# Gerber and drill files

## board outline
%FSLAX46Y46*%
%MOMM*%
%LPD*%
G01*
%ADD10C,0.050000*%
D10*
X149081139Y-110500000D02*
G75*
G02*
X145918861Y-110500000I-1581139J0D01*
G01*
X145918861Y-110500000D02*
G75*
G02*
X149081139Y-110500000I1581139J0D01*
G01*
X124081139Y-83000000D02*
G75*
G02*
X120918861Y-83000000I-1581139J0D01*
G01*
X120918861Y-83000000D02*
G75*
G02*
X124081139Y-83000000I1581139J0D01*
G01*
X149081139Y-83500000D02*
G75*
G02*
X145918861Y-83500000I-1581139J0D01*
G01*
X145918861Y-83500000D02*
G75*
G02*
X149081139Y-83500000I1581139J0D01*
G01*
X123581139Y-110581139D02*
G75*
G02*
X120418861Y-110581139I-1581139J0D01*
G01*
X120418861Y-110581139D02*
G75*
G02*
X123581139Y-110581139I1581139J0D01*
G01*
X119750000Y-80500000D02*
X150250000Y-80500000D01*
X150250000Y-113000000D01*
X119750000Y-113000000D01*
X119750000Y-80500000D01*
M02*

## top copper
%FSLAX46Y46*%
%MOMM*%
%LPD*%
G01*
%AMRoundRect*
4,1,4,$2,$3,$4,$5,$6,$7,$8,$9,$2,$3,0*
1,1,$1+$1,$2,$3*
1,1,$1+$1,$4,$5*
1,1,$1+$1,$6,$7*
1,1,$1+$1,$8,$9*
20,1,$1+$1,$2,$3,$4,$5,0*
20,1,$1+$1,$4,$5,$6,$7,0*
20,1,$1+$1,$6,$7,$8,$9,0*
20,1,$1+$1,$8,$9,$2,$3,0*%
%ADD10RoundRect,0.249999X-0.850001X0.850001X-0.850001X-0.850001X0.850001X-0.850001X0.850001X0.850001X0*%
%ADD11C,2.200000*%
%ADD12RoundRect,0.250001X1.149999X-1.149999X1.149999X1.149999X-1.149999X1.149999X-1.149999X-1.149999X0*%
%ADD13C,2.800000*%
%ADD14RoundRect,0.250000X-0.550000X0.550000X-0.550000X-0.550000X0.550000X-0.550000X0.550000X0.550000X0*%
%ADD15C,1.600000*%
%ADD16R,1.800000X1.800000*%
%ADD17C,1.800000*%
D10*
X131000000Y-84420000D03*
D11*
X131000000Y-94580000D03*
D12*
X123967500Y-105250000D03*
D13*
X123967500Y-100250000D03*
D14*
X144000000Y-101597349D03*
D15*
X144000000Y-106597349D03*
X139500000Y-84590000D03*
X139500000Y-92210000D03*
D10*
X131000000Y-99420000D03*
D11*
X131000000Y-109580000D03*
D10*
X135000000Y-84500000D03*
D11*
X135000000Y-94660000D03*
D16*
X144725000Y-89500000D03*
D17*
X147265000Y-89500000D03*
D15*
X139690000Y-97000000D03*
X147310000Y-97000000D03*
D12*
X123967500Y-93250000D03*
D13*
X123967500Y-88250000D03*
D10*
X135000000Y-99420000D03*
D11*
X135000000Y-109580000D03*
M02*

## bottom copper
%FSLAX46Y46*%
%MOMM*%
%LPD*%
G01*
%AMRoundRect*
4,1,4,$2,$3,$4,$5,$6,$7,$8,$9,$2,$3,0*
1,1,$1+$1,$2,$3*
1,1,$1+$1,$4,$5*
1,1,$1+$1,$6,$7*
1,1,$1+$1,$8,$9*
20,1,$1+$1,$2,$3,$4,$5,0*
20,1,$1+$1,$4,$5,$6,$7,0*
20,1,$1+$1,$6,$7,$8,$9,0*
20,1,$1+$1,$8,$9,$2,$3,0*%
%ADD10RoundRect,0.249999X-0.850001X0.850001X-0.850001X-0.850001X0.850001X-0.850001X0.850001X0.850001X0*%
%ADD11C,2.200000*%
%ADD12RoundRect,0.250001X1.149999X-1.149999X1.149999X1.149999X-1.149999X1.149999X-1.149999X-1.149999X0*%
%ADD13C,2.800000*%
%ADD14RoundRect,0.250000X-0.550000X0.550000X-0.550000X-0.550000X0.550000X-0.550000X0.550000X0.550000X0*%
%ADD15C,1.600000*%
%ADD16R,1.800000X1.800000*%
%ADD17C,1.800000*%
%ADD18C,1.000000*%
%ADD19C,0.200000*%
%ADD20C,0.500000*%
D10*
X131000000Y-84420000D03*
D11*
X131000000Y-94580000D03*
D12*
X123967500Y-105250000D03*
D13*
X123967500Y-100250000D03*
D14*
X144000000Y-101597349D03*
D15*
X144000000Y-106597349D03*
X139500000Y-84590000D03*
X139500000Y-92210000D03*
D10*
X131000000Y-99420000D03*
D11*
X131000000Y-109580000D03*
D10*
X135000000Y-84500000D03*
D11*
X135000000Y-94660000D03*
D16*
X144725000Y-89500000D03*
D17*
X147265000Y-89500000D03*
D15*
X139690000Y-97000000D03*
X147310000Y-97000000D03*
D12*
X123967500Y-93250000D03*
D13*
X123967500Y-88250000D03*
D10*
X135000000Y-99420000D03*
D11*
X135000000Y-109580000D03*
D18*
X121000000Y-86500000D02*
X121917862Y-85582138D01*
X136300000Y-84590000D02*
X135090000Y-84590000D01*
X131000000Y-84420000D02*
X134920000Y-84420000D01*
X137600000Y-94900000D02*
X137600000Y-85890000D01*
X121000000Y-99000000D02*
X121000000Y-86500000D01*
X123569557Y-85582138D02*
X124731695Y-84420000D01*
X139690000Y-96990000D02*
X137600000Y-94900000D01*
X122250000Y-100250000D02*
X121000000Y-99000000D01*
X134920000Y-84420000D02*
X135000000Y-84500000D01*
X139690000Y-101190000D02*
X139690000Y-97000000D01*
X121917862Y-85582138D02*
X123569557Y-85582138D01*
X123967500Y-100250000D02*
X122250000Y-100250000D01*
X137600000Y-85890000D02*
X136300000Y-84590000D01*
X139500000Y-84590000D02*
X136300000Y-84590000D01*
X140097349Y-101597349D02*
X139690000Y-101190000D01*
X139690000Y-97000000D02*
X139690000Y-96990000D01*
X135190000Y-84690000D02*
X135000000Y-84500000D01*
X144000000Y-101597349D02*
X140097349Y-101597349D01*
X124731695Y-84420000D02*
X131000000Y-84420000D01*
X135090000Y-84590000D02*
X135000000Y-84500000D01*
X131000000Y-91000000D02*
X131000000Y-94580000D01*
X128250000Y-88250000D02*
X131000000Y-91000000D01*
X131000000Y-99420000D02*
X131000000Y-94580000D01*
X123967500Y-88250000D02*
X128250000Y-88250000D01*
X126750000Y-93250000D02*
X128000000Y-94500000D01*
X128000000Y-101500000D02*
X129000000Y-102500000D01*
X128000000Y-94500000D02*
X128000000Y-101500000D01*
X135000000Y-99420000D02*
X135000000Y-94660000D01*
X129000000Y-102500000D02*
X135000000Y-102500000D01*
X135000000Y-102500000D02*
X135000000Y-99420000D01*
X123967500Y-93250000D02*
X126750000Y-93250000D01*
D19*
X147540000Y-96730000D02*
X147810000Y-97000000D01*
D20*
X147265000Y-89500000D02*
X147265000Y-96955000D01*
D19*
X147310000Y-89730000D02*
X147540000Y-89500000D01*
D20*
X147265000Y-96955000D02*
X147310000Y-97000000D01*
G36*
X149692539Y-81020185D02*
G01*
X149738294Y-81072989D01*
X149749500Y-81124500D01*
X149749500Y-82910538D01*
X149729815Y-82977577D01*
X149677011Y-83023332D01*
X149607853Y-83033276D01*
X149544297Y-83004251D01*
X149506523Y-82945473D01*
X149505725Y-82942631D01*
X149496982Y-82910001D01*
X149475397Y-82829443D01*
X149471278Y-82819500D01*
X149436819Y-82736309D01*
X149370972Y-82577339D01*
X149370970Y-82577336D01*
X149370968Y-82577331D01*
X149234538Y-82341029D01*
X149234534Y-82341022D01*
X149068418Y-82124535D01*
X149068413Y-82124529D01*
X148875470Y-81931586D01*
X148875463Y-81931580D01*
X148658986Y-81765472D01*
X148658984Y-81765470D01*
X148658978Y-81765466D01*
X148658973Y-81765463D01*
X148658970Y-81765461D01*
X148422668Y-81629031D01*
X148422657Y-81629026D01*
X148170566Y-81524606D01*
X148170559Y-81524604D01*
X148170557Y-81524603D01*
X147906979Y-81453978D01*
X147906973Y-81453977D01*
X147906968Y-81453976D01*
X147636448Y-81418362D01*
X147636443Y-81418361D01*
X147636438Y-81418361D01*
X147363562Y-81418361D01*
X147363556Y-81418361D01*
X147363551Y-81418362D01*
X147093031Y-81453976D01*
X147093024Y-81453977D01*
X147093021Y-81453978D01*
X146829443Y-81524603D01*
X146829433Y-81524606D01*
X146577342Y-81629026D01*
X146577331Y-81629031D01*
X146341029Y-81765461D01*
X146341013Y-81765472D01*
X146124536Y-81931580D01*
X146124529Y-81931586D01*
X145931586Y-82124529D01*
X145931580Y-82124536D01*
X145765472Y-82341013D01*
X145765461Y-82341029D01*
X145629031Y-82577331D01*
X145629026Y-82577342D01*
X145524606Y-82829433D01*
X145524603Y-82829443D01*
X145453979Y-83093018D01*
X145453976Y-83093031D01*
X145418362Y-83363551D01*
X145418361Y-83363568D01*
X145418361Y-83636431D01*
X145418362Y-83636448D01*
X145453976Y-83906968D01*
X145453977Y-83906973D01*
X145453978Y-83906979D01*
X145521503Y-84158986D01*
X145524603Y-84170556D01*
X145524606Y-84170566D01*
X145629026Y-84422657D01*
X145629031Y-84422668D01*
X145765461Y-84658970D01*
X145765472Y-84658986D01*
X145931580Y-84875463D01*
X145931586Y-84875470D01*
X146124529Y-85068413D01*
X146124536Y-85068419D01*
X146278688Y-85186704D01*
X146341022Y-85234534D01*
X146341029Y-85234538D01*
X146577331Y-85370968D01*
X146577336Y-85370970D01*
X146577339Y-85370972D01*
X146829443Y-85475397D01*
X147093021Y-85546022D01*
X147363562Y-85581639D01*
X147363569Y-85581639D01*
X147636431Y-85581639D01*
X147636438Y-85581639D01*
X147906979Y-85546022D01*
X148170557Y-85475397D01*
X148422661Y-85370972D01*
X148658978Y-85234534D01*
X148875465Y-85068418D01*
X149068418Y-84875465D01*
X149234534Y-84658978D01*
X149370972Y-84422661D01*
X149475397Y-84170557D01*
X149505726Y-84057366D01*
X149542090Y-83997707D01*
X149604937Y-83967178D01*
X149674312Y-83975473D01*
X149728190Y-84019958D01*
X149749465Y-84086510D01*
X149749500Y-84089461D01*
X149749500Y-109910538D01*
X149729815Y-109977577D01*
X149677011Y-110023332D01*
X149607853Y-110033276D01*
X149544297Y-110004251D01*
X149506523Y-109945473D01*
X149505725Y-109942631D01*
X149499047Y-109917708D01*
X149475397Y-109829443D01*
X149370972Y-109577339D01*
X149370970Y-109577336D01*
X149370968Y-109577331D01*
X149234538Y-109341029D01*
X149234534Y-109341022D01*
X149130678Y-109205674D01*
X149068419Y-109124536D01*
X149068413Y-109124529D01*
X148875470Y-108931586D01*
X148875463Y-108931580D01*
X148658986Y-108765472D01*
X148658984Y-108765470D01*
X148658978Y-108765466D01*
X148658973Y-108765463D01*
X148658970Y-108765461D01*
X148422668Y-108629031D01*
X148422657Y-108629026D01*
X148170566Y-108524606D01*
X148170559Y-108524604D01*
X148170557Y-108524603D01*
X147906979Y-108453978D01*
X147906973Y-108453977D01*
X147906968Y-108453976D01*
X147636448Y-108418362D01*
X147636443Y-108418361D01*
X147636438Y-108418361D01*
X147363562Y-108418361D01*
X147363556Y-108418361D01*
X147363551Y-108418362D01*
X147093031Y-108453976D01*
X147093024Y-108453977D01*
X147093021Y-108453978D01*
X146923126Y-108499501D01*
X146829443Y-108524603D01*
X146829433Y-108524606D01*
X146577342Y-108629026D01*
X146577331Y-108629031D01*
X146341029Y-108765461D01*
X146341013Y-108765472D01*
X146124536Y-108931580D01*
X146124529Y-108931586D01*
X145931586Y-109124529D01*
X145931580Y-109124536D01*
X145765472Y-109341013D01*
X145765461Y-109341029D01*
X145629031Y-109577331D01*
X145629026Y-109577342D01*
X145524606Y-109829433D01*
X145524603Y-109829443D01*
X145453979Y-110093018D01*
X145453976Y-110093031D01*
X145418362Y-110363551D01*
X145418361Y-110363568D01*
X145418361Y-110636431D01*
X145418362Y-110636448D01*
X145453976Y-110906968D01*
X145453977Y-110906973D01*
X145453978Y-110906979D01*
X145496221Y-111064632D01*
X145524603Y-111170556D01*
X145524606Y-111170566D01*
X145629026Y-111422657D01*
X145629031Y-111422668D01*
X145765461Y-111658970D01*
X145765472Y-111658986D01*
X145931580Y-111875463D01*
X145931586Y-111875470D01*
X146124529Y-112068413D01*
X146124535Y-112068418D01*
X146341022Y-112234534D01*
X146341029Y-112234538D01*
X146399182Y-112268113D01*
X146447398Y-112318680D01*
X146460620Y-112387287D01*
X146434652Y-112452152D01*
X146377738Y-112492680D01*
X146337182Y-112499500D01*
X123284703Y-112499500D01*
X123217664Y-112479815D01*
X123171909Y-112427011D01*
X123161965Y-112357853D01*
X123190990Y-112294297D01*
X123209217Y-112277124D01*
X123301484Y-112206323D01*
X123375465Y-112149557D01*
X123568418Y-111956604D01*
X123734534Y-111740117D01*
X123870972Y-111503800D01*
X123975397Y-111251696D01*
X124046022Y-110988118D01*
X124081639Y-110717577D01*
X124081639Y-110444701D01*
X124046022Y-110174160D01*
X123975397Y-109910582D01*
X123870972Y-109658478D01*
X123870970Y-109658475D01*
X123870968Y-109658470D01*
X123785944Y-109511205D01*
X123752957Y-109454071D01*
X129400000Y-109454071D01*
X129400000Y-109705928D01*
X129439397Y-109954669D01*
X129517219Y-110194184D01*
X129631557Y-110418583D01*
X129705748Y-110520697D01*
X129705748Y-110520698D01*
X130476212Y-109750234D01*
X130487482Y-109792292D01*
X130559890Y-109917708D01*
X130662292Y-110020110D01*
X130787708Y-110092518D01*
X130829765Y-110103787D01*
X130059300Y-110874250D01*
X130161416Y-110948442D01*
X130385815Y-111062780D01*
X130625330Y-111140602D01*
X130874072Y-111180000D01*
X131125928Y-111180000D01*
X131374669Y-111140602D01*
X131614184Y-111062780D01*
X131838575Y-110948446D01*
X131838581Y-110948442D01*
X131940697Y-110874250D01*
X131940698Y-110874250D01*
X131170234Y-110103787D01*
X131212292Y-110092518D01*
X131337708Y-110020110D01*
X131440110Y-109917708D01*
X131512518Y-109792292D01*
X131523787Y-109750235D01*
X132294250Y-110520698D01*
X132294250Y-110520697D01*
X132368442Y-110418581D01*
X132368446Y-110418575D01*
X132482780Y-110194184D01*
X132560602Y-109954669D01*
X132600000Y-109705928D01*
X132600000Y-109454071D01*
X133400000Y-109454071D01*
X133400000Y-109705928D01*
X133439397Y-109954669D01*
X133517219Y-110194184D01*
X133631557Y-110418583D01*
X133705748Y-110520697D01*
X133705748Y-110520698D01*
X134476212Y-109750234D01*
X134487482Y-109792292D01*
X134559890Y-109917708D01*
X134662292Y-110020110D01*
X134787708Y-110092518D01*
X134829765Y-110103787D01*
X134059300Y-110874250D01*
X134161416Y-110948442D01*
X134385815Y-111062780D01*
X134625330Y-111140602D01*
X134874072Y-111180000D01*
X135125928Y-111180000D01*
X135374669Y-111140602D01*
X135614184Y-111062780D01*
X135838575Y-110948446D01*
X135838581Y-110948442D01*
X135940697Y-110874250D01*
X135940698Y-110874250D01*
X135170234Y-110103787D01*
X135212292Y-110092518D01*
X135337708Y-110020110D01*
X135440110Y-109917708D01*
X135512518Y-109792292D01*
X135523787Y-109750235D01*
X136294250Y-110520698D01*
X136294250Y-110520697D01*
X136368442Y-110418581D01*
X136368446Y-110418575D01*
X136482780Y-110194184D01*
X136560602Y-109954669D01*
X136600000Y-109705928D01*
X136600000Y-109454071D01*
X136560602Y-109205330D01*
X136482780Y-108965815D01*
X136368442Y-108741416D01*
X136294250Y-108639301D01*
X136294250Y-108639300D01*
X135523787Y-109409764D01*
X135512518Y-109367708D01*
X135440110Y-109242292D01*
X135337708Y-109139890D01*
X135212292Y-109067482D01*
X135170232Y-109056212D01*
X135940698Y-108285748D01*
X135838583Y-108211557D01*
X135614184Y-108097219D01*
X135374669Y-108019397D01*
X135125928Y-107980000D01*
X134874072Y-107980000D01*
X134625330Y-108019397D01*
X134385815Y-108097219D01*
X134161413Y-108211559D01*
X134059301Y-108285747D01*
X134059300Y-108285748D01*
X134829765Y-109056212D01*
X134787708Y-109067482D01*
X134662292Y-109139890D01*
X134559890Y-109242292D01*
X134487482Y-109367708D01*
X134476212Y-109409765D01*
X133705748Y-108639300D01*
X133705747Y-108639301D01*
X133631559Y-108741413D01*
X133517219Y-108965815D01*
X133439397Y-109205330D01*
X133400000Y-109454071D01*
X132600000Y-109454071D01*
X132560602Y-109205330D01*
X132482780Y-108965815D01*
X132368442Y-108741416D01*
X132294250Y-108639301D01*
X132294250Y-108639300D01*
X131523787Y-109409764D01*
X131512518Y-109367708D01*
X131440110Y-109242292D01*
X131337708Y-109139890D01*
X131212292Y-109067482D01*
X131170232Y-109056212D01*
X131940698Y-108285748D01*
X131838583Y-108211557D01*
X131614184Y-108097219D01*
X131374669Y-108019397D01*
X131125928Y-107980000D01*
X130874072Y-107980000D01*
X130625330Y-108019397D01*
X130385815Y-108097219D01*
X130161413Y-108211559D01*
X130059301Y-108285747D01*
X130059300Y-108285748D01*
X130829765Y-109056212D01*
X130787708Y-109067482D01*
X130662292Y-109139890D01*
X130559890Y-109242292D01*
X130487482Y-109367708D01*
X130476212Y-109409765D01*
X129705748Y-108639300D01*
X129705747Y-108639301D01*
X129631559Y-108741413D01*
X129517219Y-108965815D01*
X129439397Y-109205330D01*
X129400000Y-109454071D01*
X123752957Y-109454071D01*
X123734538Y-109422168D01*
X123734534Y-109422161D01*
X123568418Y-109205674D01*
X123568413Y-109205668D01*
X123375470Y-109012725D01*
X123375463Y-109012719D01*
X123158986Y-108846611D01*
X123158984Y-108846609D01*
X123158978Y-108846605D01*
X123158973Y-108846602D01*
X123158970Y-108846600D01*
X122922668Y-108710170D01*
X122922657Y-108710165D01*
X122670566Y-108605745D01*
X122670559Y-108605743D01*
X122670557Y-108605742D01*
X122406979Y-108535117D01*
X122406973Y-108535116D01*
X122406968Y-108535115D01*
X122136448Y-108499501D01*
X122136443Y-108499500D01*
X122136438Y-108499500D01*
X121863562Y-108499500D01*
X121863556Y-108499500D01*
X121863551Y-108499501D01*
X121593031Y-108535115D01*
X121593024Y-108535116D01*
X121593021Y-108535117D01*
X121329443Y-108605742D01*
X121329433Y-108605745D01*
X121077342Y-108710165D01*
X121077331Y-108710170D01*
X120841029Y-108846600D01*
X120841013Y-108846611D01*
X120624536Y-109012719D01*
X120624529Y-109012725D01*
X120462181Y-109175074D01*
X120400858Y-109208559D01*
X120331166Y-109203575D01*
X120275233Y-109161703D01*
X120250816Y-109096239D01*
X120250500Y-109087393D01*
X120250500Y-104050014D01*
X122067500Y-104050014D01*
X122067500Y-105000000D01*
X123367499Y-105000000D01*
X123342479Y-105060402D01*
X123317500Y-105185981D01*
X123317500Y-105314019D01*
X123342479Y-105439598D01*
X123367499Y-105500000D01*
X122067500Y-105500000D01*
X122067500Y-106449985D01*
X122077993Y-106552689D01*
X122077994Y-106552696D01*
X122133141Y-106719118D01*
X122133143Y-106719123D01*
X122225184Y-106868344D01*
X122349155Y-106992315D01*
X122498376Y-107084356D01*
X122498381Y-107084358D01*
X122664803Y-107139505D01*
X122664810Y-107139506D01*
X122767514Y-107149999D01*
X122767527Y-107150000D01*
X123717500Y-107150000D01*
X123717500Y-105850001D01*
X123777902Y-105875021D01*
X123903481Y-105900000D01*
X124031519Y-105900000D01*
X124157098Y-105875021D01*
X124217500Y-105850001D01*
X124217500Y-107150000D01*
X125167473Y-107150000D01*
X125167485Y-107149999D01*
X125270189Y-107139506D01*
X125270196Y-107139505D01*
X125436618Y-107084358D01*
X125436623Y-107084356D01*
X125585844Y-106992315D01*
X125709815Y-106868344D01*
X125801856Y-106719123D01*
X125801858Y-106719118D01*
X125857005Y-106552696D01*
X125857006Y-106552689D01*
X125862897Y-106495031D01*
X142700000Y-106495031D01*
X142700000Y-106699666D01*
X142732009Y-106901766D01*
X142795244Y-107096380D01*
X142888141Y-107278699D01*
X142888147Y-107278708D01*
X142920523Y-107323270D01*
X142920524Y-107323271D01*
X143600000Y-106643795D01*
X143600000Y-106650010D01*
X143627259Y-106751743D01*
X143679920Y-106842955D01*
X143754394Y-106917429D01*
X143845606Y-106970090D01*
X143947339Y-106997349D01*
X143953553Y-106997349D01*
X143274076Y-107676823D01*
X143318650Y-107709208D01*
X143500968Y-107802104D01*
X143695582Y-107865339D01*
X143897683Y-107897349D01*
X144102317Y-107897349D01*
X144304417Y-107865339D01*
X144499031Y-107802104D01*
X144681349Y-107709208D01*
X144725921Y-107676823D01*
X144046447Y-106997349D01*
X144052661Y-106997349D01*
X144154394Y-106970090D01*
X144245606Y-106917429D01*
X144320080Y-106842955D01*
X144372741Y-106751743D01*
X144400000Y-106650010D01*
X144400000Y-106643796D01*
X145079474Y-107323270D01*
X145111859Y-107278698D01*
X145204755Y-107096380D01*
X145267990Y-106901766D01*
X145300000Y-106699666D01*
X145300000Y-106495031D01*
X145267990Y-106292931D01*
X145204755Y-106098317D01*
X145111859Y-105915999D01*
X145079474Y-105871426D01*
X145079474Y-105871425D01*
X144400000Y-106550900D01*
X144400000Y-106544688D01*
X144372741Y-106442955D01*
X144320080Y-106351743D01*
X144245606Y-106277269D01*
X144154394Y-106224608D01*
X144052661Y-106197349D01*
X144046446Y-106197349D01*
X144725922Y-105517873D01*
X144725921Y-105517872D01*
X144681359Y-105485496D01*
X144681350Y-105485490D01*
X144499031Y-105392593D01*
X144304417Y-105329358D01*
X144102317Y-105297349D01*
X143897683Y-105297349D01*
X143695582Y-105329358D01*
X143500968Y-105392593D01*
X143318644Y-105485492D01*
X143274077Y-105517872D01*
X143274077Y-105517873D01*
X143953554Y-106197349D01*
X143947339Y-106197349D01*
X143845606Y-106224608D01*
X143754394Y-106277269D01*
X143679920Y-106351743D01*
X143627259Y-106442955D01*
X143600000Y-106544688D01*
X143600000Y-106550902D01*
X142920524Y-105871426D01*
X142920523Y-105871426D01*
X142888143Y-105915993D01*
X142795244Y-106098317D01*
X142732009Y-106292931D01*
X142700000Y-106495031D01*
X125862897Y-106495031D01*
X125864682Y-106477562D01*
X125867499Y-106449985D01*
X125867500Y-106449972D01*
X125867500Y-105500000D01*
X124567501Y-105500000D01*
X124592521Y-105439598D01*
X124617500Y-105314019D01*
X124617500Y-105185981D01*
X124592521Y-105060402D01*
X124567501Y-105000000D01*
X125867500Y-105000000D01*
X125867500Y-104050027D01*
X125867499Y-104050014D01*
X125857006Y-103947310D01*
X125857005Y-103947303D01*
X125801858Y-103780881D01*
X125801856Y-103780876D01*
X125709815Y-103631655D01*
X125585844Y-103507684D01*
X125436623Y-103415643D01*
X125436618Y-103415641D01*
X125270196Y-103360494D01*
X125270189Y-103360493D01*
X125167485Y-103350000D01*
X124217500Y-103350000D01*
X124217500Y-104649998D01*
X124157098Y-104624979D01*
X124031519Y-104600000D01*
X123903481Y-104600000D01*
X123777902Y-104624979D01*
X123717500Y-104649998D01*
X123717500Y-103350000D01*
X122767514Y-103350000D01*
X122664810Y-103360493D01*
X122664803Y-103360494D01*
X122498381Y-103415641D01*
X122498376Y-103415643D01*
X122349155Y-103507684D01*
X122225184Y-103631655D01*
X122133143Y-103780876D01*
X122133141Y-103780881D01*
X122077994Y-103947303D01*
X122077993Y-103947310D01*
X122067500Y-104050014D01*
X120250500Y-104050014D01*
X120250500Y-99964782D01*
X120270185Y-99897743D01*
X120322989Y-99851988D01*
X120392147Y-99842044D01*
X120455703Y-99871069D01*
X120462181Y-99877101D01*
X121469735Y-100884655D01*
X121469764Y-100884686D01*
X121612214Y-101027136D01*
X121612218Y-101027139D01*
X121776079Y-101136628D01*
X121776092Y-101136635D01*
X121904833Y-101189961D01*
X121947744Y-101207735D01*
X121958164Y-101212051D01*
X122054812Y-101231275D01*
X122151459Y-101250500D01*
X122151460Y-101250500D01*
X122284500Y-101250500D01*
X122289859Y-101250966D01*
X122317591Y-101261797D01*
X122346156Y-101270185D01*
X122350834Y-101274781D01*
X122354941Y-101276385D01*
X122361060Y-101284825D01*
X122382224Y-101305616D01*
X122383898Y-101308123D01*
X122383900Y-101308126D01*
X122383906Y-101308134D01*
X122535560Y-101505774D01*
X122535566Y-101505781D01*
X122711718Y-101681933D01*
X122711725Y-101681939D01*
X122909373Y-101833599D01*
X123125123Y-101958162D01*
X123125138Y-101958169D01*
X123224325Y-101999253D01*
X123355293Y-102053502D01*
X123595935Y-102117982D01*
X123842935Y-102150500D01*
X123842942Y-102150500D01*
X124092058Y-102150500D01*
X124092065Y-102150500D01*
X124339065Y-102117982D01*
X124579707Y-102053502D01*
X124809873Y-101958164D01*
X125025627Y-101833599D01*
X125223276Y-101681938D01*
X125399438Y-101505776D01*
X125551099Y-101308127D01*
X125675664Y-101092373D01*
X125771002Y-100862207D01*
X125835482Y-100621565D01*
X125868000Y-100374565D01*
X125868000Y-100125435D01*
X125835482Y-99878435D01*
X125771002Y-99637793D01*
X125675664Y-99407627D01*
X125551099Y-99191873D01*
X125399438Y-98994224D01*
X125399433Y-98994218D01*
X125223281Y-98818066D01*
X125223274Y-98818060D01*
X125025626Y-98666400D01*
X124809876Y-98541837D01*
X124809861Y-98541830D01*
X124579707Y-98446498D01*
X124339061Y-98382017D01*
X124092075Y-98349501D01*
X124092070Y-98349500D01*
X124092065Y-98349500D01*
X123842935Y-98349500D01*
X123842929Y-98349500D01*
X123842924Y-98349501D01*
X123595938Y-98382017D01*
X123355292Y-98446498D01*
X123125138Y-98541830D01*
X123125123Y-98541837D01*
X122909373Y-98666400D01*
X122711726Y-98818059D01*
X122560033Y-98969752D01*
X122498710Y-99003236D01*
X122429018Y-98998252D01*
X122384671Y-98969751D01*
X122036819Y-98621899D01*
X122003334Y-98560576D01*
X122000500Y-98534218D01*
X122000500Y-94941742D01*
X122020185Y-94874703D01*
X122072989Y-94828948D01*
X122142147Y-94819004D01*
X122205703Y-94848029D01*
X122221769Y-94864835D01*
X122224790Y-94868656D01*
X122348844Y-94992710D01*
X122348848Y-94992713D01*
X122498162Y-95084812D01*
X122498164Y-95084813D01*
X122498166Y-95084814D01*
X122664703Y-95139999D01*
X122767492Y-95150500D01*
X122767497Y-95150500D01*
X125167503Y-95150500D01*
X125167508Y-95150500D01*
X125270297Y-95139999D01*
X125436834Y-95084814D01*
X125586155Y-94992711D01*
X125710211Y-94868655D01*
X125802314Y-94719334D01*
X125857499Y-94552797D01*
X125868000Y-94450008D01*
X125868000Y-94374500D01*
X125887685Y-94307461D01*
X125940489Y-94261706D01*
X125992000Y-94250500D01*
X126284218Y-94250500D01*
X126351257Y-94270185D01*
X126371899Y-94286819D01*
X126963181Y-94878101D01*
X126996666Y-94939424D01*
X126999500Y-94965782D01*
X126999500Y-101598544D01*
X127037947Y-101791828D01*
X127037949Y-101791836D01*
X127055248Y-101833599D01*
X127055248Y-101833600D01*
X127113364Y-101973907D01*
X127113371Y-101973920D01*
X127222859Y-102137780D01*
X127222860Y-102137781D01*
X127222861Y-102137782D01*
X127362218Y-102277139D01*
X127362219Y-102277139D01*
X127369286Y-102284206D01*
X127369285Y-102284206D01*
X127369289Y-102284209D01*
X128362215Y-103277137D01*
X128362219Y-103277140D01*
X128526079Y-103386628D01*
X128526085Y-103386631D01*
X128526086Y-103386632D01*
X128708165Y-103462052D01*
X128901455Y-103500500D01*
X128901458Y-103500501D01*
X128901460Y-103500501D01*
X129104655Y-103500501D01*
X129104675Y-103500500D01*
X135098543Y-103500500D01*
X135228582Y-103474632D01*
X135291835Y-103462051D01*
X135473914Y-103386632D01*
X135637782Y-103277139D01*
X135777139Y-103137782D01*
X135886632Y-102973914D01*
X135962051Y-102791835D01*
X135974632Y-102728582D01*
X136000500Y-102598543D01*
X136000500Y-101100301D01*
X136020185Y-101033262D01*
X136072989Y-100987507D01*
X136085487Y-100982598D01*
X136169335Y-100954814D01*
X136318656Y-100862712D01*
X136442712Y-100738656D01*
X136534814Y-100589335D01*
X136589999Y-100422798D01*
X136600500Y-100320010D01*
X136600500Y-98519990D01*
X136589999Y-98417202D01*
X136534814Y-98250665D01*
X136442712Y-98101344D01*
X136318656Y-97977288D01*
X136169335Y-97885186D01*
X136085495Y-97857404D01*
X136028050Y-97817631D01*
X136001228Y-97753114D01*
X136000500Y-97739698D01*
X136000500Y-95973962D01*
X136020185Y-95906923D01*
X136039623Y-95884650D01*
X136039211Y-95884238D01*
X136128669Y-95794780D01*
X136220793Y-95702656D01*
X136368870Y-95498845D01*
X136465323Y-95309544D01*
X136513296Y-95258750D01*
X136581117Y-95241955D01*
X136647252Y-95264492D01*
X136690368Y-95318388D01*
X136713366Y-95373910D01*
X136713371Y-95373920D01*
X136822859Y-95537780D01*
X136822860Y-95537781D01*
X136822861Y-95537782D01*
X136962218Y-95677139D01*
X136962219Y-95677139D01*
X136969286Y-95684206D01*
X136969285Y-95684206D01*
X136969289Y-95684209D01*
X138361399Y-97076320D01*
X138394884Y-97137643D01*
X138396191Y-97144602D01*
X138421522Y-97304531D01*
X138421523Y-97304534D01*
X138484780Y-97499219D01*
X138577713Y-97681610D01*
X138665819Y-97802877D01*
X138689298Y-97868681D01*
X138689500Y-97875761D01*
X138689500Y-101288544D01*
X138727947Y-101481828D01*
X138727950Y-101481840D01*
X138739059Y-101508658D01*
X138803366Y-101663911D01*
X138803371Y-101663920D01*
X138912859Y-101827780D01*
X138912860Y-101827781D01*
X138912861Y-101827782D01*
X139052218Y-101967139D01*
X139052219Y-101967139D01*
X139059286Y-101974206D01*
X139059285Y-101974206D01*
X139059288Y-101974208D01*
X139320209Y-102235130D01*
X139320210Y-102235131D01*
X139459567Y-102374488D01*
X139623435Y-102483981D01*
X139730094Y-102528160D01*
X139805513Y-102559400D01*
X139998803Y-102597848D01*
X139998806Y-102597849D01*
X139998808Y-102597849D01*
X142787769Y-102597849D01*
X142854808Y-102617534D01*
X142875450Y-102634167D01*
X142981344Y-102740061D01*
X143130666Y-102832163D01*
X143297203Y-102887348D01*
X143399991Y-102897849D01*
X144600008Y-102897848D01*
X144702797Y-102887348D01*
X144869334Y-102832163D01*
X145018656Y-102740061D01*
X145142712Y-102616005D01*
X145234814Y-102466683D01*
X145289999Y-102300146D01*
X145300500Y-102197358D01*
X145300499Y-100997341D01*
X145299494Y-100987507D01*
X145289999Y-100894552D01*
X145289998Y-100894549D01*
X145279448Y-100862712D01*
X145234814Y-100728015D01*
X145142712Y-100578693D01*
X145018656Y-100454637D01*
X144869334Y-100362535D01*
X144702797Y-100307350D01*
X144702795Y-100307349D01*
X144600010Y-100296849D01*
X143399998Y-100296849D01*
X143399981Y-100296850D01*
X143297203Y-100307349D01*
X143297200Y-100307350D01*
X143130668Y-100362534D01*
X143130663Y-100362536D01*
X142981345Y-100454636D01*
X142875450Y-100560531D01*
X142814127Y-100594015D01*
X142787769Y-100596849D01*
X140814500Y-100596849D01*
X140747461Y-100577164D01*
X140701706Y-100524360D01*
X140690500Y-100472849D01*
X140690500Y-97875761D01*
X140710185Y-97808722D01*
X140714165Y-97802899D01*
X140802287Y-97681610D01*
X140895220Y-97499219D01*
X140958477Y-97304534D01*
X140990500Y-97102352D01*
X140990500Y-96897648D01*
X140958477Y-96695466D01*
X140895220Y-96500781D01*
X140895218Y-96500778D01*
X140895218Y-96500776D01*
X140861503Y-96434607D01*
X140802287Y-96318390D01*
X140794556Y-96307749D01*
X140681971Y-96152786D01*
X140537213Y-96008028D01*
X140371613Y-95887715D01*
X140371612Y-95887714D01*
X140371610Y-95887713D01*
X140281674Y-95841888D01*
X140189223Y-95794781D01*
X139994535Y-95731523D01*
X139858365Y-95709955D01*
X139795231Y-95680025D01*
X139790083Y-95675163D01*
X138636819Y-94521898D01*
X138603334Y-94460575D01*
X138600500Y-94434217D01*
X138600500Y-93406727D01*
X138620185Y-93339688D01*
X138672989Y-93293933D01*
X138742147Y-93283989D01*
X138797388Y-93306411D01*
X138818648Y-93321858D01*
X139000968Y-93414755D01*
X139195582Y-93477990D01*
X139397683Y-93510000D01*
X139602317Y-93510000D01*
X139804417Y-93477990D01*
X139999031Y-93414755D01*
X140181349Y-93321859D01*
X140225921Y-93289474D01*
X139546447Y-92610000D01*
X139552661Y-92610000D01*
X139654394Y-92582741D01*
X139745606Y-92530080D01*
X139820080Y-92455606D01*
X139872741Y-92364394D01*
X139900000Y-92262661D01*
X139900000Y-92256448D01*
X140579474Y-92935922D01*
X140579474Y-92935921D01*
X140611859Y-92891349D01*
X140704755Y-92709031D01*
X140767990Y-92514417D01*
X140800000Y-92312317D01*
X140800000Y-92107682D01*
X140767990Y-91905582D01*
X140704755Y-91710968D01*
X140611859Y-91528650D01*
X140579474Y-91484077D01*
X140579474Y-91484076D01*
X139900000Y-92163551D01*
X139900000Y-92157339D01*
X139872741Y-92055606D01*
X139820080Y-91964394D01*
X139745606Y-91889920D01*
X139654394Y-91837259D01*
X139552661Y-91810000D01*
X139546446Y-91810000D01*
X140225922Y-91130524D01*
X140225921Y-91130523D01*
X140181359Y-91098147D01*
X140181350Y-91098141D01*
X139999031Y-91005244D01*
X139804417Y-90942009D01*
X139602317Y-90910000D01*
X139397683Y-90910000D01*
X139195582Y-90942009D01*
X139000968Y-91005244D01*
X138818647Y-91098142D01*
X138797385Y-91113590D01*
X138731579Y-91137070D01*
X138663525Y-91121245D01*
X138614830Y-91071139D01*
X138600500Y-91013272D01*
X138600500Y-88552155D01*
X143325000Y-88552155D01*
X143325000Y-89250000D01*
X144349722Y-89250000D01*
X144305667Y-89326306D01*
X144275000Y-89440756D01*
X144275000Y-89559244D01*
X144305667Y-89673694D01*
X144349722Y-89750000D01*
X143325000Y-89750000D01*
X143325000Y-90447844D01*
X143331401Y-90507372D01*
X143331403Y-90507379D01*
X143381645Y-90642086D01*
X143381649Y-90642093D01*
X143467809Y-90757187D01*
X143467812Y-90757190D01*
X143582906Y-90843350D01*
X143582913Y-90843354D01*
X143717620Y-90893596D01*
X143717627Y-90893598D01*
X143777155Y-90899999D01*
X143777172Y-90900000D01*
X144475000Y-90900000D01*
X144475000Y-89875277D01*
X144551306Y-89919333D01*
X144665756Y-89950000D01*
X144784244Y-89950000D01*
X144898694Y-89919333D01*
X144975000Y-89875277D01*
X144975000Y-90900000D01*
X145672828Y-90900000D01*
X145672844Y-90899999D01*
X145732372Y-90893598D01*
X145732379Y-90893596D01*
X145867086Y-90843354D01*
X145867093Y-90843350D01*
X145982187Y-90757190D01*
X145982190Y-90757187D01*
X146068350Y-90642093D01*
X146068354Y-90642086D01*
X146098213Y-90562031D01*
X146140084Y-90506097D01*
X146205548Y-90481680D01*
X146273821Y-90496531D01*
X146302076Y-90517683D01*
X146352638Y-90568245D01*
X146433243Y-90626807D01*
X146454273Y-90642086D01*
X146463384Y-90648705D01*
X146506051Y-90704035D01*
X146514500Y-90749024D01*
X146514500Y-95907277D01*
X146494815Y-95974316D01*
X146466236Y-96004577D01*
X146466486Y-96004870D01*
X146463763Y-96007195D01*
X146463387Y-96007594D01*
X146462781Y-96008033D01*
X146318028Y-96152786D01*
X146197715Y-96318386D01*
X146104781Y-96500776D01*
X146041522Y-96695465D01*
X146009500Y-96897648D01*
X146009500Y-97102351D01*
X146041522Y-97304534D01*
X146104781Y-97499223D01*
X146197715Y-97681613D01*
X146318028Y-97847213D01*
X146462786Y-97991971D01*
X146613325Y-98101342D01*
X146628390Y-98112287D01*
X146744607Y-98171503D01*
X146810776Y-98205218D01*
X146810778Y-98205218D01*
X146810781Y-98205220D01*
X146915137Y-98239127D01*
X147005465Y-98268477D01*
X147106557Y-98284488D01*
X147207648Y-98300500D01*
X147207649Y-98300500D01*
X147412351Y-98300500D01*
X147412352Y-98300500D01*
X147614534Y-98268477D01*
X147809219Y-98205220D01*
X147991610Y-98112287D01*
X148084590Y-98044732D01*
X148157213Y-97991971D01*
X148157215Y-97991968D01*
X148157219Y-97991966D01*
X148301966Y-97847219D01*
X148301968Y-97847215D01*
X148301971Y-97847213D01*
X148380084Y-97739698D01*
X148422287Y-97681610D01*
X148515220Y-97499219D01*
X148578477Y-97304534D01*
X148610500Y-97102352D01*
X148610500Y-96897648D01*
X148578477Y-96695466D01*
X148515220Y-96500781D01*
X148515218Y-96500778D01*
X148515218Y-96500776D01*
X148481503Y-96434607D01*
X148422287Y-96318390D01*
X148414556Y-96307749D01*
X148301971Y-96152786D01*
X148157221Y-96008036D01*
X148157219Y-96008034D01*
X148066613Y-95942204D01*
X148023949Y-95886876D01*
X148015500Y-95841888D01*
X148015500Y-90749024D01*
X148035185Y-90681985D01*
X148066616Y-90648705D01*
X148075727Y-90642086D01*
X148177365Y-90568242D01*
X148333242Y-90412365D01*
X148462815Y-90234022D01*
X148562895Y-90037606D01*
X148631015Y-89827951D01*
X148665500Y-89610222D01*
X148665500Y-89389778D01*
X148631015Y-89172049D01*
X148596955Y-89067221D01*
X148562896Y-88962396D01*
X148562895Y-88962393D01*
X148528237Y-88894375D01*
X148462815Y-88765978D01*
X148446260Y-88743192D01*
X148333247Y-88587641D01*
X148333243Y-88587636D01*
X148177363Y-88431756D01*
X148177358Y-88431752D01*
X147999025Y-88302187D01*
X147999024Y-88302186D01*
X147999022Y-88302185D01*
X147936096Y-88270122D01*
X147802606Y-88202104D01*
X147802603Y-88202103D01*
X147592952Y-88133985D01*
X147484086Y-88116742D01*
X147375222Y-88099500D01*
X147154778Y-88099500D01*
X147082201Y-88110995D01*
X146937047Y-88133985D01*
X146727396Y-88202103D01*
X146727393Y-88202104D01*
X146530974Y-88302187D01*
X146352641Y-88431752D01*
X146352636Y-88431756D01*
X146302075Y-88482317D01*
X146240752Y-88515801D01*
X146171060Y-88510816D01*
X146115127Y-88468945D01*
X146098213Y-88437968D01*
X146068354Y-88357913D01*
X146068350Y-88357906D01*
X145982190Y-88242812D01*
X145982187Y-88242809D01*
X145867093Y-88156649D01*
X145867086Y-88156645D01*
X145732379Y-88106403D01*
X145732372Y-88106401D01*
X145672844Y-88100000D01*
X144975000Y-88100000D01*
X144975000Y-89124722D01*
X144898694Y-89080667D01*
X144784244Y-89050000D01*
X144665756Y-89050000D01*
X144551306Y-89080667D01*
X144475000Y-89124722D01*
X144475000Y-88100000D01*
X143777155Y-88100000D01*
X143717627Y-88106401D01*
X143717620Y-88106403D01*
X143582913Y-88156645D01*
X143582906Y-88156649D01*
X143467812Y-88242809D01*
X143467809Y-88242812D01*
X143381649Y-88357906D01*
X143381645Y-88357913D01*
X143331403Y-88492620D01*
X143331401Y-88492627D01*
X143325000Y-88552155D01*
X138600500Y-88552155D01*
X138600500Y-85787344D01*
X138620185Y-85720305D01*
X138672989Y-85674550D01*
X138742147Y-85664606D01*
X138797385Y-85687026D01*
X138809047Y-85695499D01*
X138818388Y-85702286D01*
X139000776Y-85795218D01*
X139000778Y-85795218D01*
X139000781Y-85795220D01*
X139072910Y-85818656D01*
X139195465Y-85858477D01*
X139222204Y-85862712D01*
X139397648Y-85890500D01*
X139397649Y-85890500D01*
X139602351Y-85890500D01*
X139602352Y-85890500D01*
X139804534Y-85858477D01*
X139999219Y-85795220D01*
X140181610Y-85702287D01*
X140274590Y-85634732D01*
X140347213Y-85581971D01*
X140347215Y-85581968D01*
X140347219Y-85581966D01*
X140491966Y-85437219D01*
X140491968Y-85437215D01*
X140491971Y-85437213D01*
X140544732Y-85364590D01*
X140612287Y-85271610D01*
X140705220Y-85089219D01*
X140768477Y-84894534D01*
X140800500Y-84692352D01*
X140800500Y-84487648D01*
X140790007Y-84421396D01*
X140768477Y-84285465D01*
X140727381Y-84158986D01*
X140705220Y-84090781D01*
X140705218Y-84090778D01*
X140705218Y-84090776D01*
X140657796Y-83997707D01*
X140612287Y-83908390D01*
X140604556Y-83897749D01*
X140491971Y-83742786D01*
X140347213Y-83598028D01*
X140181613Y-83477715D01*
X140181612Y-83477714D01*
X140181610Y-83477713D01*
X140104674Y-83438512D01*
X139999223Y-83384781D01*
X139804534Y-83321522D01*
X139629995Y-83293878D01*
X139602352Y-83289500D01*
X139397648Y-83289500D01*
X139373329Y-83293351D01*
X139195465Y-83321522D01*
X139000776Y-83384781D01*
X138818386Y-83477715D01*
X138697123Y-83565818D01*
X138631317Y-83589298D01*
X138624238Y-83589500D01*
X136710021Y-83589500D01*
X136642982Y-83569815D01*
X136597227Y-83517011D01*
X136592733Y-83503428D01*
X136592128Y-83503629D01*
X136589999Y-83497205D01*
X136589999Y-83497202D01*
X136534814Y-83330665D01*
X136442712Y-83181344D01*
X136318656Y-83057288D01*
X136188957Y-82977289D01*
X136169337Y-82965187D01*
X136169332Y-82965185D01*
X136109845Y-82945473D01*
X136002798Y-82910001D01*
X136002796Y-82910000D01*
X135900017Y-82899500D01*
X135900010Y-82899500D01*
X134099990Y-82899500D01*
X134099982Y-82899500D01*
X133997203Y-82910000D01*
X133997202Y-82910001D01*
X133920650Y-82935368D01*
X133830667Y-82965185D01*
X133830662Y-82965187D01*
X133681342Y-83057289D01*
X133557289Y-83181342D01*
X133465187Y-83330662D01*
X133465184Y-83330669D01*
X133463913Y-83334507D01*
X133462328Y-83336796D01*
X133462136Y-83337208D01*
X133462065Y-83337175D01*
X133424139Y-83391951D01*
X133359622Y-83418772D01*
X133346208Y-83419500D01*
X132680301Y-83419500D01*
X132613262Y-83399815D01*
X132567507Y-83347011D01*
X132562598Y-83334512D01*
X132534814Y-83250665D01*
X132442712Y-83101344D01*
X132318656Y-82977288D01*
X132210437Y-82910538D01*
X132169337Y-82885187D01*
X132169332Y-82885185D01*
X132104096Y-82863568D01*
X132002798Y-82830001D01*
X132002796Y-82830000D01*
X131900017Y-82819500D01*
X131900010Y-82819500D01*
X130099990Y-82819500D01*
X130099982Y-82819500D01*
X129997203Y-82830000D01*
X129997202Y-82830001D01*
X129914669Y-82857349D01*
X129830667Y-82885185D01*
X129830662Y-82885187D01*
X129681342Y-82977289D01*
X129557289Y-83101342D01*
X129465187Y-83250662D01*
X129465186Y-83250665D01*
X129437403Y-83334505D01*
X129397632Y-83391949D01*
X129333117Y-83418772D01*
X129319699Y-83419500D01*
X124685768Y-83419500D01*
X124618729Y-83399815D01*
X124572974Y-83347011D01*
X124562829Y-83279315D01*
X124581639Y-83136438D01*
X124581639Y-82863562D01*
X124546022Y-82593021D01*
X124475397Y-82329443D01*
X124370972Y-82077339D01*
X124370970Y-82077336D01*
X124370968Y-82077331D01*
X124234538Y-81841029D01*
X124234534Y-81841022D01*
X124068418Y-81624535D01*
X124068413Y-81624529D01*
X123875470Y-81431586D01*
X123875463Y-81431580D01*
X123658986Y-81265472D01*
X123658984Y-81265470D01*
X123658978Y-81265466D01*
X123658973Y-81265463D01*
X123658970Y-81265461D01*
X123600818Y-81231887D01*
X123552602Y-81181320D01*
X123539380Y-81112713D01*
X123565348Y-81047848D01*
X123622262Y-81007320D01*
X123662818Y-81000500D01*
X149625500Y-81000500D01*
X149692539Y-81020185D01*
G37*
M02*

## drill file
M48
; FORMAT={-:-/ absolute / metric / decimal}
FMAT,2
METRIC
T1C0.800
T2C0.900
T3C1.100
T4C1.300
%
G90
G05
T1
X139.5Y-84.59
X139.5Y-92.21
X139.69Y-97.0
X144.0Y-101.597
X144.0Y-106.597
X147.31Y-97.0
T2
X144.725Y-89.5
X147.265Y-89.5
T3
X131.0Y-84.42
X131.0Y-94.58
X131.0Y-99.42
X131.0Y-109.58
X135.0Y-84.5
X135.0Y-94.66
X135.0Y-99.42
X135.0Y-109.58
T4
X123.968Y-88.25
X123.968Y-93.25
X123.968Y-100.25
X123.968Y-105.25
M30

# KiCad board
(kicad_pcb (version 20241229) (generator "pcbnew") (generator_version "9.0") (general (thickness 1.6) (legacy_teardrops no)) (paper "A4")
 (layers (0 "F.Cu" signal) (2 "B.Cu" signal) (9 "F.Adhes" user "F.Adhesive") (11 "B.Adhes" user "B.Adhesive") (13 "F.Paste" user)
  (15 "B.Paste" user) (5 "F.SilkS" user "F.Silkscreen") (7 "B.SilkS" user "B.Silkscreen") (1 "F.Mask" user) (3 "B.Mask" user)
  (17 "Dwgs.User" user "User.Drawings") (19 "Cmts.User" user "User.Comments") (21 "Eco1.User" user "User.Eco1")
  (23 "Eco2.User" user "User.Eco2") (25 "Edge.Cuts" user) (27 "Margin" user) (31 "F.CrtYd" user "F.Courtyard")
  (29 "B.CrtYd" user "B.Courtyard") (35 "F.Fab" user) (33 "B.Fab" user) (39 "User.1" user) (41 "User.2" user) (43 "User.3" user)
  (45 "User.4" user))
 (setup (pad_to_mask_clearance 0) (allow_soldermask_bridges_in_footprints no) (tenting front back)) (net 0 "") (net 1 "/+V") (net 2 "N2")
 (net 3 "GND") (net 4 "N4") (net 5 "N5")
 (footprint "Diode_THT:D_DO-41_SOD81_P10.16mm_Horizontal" (layer "F.Cu") (at 131 84.42 -90)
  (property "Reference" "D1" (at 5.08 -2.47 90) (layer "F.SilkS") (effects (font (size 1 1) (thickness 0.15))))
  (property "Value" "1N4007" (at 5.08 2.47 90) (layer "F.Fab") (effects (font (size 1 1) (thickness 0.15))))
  (pad "1" thru_hole roundrect (at 0 0 270) (size 2.2 2.2) (drill 1.1) (layers "*.Cu" "*.Mask") (remove_unused_layers no)
   (roundrect_rratio 0.113636) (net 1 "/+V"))
  (pad "2" thru_hole circle (at 10.16 0 270) (size 2.2 2.2) (drill 1.1) (layers "*.Cu" "*.Mask") (remove_unused_layers no) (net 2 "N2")))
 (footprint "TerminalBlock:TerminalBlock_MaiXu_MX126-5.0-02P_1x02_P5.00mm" (layer "F.Cu") (at 123.9675 105.25 90)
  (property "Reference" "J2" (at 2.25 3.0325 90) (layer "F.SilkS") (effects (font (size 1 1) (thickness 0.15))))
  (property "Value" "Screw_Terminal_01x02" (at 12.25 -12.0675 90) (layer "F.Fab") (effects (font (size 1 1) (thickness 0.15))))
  (pad "1" thru_hole roundrect (at 0 0 90) (size 2.8 2.8) (drill 1.3) (layers "*.Cu" "*.Mask") (remove_unused_layers no)
   (roundrect_rratio 0.089286) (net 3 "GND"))
  (pad "2" thru_hole circle (at 5 0 90) (size 2.8 2.8) (drill 1.3) (layers "*.Cu" "*.Mask") (remove_unused_layers no) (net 1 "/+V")))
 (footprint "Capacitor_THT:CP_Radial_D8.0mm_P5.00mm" (layer "F.Cu") (at 144 101.597349 -90)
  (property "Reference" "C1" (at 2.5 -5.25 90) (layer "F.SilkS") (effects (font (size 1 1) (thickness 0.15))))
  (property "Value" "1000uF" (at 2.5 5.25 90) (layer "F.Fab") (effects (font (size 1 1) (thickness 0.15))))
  (pad "1" thru_hole roundrect (at 0 0 270) (size 1.6 1.6) (drill 0.8) (layers "*.Cu" "*.Mask") (remove_unused_layers no)
   (roundrect_rratio 0.15625) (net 1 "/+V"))
  (pad "2" thru_hole circle (at 5 0 270) (size 1.6 1.6) (drill 0.8) (layers "*.Cu" "*.Mask") (remove_unused_layers no) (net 3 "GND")))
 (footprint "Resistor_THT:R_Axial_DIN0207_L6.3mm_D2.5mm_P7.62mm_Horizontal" (layer "F.Cu") (at 139.5 84.59 -90)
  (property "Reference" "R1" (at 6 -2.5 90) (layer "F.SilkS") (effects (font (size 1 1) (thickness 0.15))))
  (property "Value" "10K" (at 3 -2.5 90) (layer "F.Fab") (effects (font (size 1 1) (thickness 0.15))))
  (pad "1" thru_hole circle (at 0 0 270) (size 1.6 1.6) (drill 0.8) (layers "*.Cu" "*.Mask") (remove_unused_layers no) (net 1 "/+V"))
  (pad "2" thru_hole circle (at 7.62 0 270) (size 1.6 1.6) (drill 0.8) (layers "*.Cu" "*.Mask") (remove_unused_layers no) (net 3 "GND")))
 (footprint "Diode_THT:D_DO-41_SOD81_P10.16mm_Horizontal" (layer "F.Cu") (at 131 99.42 -90)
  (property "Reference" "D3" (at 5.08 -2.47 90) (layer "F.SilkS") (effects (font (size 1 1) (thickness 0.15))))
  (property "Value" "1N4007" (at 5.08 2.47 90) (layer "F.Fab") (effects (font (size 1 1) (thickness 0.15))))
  (pad "1" thru_hole roundrect (at 0 0 270) (size 2.2 2.2) (drill 1.1) (layers "*.Cu" "*.Mask") (remove_unused_layers no)
   (roundrect_rratio 0.113636) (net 2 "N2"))
  (pad "2" thru_hole circle (at 10.16 0 270) (size 2.2 2.2) (drill 1.1) (layers "*.Cu" "*.Mask") (remove_unused_layers no) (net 3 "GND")))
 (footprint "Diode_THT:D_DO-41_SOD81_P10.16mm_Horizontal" (layer "F.Cu") (at 135 84.5 -90)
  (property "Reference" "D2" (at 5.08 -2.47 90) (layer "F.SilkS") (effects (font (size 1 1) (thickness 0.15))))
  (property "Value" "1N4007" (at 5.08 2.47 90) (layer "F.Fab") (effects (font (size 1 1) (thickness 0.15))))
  (pad "1" thru_hole roundrect (at 0 0 270) (size 2.2 2.2) (drill 1.1) (layers "*.Cu" "*.Mask") (remove_unused_layers no)
   (roundrect_rratio 0.113636) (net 1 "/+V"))
  (pad "2" thru_hole circle (at 10.16 0 270) (size 2.2 2.2) (drill 1.1) (layers "*.Cu" "*.Mask") (remove_unused_layers no) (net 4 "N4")))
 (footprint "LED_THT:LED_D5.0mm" (layer "F.Cu") (at 144.725 89.5)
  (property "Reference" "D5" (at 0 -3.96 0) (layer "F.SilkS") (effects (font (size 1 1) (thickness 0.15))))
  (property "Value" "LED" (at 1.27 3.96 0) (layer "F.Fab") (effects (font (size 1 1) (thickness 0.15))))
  (pad "1" thru_hole rect (at 0 0) (size 1.8 1.8) (drill 0.9) (layers "*.Cu" "*.Mask") (remove_unused_layers no) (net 3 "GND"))
  (pad "2" thru_hole circle (at 2.54 0) (size 1.8 1.8) (drill 0.9) (layers "*.Cu" "*.Mask") (remove_unused_layers no) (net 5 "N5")))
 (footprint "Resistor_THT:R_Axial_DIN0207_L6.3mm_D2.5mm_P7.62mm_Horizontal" (layer "F.Cu") (at 139.69 97)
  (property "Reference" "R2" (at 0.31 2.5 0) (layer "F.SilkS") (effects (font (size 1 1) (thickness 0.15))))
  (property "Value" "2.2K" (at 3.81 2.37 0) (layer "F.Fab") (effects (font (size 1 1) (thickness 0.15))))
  (pad "1" thru_hole circle (at 0 0) (size 1.6 1.6) (drill 0.8) (layers "*.Cu" "*.Mask") (remove_unused_layers no) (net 1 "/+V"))
  (pad "2" thru_hole circle (at 7.62 0) (size 1.6 1.6) (drill 0.8) (layers "*.Cu" "*.Mask") (remove_unused_layers no) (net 5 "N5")))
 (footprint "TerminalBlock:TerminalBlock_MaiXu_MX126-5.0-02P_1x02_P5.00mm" (layer "F.Cu") (at 123.9675 93.25 90)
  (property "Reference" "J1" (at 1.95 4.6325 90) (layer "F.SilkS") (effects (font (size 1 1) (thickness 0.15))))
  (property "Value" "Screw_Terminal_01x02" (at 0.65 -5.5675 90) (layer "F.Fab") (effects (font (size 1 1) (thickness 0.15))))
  (pad "1" thru_hole roundrect (at 0 0 90) (size 2.8 2.8) (drill 1.3) (layers "*.Cu" "*.Mask") (remove_unused_layers no)
   (roundrect_rratio 0.089286) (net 4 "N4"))
  (pad "2" thru_hole circle (at 5 0 90) (size 2.8 2.8) (drill 1.3) (layers "*.Cu" "*.Mask") (remove_unused_layers no) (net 2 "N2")))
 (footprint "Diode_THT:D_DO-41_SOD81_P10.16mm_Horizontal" (layer "F.Cu") (at 135 99.42 -90)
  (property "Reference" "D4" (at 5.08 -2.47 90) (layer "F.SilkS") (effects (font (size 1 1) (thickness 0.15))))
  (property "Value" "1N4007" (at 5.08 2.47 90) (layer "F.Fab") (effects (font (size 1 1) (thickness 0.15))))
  (pad "1" thru_hole roundrect (at 0 0 270) (size 2.2 2.2) (drill 1.1) (layers "*.Cu" "*.Mask") (remove_unused_layers no)
   (roundrect_rratio 0.113636) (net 4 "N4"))
  (pad "2" thru_hole circle (at 10.16 0 270) (size 2.2 2.2) (drill 1.1) (layers "*.Cu" "*.Mask") (remove_unused_layers no) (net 3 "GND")))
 (gr_circle (center 147.5 110.5) (end 146 111) (stroke (width 0.05) (type default)) (fill no) (layer "Edge.Cuts"))
 (gr_circle (center 122.5 83) (end 121 83.5) (stroke (width 0.05) (type default)) (fill no) (layer "Edge.Cuts"))
 (gr_circle (center 147.5 83.5) (end 146 84) (stroke (width 0.05) (type default)) (fill no) (layer "Edge.Cuts"))
 (gr_circle (center 122 110.581139) (end 120.5 111.081139) (stroke (width 0.05) (type default)) (fill no) (layer "Edge.Cuts"))
 (gr_rect (start 119.75 80.5) (end 150.25 113) (stroke (width 0.05) (type default)) (fill no) (layer "Edge.Cuts"))
 (segment (start 121 86.5) (end 121.917862 85.582138) (width 1) (layer "B.Cu") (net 1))
 (segment (start 136.3 84.59) (end 135.09 84.59) (width 1) (layer "B.Cu") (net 1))
 (segment (start 131 84.42) (end 134.92 84.42) (width 1) (layer "B.Cu") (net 1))
 (segment (start 137.6 94.9) (end 137.6 85.89) (width 1) (layer "B.Cu") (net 1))
 (segment (start 121 99) (end 121 86.5) (width 1) (layer "B.Cu") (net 1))
 (segment (start 123.569557 85.582138) (end 124.731695 84.42) (width 1) (layer "B.Cu") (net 1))
 (segment (start 139.69 96.99) (end 137.6 94.9) (width 1) (layer "B.Cu") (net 1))
 (segment (start 122.25 100.25) (end 121 99) (width 1) (layer "B.Cu") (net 1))
 (segment (start 134.92 84.42) (end 135 84.5) (width 1) (layer "B.Cu") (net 1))
 (segment (start 139.69 101.19) (end 139.69 97) (width 1) (layer "B.Cu") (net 1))
 (segment (start 121.917862 85.582138) (end 123.569557 85.582138) (width 1) (layer "B.Cu") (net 1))
 (segment (start 123.9675 100.25) (end 122.25 100.25) (width 1) (layer "B.Cu") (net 1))
 (segment (start 137.6 85.89) (end 136.3 84.59) (width 1) (layer "B.Cu") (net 1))
 (segment (start 139.5 84.59) (end 136.3 84.59) (width 1) (layer "B.Cu") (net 1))
 (segment (start 140.097349 101.597349) (end 139.69 101.19) (width 1) (layer "B.Cu") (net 1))
 (segment (start 139.69 97) (end 139.69 96.99) (width 1) (layer "B.Cu") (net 1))
 (segment (start 135.19 84.69) (end 135 84.5) (width 1) (layer "B.Cu") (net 1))
 (segment (start 144 101.597349) (end 140.097349 101.597349) (width 1) (layer "B.Cu") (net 1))
 (segment (start 124.731695 84.42) (end 131 84.42) (width 1) (layer "B.Cu") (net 1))
 (segment (start 135.09 84.59) (end 135 84.5) (width 1) (layer "B.Cu") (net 1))
 (segment (start 131 91) (end 131 94.58) (width 1) (layer "B.Cu") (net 2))
 (segment (start 128.25 88.25) (end 131 91) (width 1) (layer "B.Cu") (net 2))
 (segment (start 131 99.42) (end 131 94.58) (width 1) (layer "B.Cu") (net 2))
 (segment (start 123.9675 88.25) (end 128.25 88.25) (width 1) (layer "B.Cu") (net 2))
 (segment (start 126.75 93.25) (end 128 94.5) (width 1) (layer "B.Cu") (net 4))
 (segment (start 128 101.5) (end 129 102.5) (width 1) (layer "B.Cu") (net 4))
 (segment (start 128 94.5) (end 128 101.5) (width 1) (layer "B.Cu") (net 4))
 (segment (start 135 99.42) (end 135 94.66) (width 1) (layer "B.Cu") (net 4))
 (segment (start 129 102.5) (end 135 102.5) (width 1) (layer "B.Cu") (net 4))
 (segment (start 135 102.5) (end 135 99.42) (width 1) (layer "B.Cu") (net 4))
 (segment (start 123.9675 93.25) (end 126.75 93.25) (width 1) (layer "B.Cu") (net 4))
 (segment (start 147.54 96.73) (end 147.81 97) (width 0.2) (layer "B.Cu") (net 5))
 (segment (start 147.265 89.5) (end 147.265 96.955) (width 0.5) (layer "B.Cu") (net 5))
 (segment (start 147.31 89.73) (end 147.54 89.5) (width 0.2) (layer "B.Cu") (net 5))
 (segment (start 147.265 96.955) (end 147.31 97) (width 0.5) (layer "B.Cu") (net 5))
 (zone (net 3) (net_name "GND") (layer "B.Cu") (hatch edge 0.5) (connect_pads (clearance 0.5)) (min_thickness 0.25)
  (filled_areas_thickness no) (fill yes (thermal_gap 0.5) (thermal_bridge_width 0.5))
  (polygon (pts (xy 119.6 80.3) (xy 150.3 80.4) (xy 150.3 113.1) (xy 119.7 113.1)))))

